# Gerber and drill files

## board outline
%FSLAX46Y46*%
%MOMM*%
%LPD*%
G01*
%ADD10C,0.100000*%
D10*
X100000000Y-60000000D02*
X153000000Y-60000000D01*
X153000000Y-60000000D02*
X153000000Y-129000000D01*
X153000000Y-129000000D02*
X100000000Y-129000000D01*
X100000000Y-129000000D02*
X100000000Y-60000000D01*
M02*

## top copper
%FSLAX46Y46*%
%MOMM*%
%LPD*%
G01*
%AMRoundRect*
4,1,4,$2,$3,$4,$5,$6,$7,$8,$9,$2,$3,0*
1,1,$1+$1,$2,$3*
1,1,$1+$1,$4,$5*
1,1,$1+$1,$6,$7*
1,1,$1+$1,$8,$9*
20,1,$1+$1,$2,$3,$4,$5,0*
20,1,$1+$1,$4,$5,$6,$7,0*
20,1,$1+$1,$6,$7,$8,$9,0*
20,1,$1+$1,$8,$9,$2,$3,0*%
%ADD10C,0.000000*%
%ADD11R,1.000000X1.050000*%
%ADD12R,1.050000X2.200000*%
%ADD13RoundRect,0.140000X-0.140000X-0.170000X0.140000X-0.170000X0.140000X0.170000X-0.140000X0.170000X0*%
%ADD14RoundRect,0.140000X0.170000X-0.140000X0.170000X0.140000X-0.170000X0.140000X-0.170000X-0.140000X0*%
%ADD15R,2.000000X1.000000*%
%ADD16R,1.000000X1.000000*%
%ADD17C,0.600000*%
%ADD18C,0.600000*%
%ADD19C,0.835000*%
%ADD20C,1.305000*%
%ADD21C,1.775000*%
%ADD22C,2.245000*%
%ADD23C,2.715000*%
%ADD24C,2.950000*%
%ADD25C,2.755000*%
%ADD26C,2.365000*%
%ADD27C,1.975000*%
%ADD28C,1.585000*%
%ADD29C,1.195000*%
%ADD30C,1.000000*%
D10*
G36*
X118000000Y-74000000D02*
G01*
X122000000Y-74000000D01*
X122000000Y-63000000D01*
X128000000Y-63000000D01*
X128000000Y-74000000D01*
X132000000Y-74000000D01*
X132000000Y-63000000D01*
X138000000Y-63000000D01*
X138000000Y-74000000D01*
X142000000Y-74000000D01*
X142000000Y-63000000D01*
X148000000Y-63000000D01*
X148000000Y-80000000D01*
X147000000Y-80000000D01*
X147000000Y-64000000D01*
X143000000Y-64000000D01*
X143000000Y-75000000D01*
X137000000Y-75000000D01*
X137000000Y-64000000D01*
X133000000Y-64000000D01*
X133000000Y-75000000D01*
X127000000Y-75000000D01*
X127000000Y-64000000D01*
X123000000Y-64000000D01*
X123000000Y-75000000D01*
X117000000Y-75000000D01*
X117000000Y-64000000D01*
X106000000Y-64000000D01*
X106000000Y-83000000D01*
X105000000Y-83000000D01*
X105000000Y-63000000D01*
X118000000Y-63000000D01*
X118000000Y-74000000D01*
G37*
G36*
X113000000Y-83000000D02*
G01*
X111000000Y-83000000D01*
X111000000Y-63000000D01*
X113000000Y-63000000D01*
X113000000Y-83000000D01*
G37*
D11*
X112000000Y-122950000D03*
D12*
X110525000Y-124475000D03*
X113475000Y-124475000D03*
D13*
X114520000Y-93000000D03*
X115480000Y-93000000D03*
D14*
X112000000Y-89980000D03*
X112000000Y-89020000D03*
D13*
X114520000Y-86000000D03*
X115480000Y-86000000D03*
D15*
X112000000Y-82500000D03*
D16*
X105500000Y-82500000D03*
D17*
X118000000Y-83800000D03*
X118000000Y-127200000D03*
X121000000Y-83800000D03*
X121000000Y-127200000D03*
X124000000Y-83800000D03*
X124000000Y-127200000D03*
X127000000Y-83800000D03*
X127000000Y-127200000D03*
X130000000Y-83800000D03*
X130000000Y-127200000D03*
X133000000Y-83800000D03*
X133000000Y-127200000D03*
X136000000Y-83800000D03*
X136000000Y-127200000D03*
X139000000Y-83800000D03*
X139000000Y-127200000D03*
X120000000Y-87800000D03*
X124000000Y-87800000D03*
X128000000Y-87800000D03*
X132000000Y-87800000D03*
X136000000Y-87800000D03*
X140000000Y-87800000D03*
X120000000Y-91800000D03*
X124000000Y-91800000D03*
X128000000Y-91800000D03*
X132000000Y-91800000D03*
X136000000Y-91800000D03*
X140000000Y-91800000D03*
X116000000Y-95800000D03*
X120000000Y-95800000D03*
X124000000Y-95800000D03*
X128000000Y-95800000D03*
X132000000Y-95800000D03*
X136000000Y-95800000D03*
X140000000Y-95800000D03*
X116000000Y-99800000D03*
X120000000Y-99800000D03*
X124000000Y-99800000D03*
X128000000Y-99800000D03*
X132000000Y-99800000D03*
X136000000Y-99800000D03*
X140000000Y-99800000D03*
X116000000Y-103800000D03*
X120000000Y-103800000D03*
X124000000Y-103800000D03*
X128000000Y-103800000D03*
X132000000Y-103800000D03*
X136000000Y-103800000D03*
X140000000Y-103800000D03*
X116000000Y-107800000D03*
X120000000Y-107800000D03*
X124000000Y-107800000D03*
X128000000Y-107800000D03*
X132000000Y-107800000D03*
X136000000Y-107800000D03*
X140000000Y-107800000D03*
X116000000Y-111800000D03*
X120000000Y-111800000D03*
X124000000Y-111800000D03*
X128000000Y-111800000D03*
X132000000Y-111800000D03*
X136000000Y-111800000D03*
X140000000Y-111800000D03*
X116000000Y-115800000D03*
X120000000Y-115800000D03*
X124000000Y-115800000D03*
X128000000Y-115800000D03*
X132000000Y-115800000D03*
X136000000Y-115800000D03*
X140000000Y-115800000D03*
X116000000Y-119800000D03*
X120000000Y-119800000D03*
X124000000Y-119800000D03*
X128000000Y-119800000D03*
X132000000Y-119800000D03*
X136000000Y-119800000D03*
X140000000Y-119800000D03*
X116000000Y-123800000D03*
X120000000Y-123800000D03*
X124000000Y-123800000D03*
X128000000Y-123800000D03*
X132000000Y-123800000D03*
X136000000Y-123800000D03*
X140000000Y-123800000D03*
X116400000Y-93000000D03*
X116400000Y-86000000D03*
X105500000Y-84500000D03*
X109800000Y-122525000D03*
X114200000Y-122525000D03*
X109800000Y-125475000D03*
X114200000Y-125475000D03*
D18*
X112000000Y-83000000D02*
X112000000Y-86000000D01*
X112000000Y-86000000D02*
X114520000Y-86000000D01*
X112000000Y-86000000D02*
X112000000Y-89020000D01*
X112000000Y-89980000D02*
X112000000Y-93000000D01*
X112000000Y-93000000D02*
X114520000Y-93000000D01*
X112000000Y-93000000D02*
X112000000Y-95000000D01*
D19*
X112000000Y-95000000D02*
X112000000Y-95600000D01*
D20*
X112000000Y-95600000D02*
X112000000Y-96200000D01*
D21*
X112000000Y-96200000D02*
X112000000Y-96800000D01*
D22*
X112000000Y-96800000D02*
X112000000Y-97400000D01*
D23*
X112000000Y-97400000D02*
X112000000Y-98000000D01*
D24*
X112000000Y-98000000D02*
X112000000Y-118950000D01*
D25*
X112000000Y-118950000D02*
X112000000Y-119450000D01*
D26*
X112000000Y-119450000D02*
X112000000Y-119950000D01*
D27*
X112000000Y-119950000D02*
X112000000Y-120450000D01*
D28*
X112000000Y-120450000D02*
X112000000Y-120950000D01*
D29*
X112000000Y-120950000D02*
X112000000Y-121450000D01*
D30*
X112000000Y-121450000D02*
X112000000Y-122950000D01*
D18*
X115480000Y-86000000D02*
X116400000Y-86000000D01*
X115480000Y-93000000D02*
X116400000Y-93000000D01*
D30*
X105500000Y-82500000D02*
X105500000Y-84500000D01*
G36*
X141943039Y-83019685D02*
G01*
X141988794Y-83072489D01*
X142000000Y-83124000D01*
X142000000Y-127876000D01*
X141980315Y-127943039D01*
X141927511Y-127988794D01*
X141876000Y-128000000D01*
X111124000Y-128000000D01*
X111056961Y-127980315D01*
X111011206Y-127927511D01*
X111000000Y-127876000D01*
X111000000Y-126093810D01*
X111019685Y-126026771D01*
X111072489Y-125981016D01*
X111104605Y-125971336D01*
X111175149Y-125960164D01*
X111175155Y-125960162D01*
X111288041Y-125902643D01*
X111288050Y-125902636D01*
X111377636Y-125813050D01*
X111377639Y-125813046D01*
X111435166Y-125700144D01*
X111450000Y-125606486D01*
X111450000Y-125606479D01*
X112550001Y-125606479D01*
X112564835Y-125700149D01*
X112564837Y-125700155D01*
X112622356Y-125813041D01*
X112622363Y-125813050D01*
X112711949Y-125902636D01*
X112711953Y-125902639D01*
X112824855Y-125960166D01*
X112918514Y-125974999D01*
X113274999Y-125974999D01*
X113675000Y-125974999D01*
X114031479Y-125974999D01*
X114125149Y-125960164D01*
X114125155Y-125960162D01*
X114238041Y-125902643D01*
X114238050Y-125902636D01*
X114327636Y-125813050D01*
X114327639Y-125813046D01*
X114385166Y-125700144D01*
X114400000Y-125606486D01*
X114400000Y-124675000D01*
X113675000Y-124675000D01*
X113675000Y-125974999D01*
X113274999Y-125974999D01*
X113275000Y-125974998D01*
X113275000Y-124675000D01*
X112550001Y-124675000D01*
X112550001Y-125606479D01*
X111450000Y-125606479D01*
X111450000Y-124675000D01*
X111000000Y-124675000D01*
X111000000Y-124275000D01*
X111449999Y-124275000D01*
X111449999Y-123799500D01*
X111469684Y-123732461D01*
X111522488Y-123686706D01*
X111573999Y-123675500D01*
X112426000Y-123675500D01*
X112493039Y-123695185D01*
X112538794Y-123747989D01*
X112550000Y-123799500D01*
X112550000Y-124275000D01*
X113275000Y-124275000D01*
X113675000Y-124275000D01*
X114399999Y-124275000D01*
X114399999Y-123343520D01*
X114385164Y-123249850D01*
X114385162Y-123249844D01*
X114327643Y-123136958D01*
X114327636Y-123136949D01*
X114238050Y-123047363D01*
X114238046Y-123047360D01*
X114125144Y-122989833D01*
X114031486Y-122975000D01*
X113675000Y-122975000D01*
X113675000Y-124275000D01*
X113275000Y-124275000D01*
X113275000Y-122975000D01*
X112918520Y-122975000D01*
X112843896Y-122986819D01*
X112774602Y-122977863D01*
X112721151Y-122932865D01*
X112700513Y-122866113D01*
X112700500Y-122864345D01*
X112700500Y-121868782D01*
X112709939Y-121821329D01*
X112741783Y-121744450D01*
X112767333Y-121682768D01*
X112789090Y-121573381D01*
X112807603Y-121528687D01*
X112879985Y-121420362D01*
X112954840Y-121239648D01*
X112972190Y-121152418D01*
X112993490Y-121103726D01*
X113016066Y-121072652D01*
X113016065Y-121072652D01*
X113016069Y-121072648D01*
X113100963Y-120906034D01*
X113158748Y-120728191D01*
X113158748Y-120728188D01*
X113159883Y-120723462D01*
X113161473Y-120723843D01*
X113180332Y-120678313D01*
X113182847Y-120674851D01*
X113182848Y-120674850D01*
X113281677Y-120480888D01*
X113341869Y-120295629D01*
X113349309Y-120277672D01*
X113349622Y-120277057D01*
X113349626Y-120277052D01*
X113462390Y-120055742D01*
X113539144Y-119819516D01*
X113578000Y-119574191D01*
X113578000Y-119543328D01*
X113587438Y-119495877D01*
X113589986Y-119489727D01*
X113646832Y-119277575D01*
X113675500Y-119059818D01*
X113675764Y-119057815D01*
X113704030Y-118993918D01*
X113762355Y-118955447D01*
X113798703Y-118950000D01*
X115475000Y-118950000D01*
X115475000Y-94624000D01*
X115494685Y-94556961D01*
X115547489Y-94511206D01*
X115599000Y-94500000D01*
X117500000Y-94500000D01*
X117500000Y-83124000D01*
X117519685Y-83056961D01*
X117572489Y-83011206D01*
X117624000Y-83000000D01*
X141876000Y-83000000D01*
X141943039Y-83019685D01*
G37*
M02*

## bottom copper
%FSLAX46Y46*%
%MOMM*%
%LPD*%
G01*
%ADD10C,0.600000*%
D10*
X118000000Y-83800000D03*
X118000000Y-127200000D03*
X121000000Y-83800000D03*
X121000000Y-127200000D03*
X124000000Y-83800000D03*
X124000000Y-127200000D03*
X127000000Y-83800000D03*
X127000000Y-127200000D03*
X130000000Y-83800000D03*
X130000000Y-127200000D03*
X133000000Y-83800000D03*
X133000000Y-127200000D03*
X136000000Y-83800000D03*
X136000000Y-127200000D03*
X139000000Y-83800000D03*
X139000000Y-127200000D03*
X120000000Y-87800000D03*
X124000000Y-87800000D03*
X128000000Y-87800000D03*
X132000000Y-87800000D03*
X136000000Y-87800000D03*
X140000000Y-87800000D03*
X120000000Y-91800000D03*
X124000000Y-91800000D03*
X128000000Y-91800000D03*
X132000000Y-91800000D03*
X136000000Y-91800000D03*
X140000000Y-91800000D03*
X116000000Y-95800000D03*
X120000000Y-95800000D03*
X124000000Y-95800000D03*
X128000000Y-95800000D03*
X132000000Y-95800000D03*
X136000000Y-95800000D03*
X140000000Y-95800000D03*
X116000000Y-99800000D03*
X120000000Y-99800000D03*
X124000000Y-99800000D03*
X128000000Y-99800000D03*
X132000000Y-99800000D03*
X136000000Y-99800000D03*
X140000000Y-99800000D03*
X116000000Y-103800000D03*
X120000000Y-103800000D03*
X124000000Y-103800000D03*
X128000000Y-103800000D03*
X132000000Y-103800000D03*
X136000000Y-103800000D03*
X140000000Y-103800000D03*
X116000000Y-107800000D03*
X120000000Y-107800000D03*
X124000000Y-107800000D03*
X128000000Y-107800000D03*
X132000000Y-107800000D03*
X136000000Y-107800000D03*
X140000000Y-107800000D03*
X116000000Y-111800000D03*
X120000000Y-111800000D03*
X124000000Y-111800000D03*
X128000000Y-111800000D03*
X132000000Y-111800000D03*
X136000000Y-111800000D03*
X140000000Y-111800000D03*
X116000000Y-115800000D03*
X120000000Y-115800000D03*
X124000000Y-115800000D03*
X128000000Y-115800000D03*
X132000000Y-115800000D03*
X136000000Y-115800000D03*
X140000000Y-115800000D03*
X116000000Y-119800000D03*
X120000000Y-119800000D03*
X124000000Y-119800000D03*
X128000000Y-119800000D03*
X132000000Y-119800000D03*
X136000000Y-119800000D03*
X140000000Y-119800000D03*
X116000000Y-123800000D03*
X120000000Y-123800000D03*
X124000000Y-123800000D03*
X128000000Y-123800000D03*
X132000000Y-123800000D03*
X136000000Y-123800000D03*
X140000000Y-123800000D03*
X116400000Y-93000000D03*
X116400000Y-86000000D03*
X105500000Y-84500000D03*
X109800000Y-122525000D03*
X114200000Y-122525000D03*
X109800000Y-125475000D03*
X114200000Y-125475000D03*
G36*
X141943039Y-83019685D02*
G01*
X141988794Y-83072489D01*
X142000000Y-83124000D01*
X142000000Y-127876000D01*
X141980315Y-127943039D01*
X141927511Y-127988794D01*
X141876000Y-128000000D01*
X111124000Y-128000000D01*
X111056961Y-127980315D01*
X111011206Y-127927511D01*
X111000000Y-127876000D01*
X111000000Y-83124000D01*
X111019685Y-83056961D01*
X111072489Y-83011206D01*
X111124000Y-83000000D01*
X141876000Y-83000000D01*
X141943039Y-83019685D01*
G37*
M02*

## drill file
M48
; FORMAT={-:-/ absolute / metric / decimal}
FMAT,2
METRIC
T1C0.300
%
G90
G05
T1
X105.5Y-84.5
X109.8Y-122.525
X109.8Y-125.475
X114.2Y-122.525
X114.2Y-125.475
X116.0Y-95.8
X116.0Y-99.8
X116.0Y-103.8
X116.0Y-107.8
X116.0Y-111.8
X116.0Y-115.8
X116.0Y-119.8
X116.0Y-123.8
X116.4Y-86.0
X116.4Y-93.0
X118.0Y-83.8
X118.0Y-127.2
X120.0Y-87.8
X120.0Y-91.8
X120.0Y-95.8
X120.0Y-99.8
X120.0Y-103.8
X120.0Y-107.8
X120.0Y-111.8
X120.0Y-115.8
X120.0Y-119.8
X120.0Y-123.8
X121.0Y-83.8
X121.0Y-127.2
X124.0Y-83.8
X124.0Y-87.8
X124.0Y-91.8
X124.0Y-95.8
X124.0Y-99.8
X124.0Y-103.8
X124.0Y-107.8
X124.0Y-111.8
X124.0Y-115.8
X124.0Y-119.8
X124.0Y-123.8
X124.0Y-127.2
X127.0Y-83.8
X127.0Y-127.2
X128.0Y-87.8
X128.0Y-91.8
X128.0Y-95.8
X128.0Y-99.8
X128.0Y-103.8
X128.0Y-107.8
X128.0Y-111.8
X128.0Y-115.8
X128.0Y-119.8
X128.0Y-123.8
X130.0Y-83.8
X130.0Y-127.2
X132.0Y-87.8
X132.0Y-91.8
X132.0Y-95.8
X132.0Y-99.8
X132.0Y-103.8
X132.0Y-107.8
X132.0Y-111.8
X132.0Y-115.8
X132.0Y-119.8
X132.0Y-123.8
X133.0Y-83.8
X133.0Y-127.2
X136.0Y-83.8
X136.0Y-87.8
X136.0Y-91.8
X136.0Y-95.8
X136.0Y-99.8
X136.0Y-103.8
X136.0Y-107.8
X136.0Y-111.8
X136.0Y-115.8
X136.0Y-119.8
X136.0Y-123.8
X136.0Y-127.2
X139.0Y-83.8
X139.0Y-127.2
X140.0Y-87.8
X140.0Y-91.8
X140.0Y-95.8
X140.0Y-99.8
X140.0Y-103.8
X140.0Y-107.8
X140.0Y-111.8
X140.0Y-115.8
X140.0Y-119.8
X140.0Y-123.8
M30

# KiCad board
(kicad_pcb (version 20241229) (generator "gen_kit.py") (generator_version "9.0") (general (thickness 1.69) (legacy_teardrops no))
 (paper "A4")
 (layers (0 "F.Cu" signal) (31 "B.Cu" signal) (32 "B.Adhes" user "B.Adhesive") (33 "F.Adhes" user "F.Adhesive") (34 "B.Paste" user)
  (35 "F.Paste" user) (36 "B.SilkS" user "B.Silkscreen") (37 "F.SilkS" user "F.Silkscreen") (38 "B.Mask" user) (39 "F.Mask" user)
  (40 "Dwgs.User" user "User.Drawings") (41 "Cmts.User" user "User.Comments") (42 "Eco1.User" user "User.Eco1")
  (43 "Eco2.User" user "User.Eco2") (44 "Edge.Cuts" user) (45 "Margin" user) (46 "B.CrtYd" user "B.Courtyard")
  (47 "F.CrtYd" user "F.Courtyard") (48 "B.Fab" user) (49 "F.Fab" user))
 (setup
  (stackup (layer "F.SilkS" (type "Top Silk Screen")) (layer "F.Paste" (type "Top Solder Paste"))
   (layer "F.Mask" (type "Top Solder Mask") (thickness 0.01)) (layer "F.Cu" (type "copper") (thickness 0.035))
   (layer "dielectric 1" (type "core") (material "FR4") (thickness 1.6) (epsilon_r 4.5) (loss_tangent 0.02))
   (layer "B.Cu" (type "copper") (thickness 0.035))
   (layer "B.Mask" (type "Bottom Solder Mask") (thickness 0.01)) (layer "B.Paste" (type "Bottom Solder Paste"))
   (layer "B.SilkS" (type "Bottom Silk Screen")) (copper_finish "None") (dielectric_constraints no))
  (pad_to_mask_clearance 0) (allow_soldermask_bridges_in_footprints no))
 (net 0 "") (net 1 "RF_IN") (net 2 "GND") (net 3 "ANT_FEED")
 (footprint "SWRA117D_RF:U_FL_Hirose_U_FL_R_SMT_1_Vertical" (layer "F.Cu") (at 112 124 270)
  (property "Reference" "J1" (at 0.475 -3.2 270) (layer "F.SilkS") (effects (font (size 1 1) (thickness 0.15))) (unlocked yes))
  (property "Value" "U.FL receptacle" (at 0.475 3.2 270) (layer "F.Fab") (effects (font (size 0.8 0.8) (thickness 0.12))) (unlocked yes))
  (pad "1" smd rect (at -1.05 0 270) (size 1.05 1) (layers "F.Cu" "F.Paste" "F.Mask") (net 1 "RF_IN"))
  (pad "2" smd rect (at 0.475 1.475 270) (size 2.2 1.05) (layers "F.Cu" "F.Paste" "F.Mask") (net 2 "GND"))
  (pad "2" smd rect (at 0.475 -1.475 270) (size 2.2 1.05) (layers "F.Cu" "F.Paste" "F.Mask") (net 2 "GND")))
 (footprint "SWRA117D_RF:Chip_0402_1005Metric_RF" (layer "F.Cu") (at 115 93)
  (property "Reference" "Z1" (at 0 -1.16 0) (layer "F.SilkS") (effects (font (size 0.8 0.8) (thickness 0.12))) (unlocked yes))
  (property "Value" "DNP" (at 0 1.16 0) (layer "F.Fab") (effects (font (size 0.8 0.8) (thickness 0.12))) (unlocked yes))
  (pad "1" smd roundrect (at -0.48 0) (size 0.56 0.62) (layers "F.Cu" "F.Paste" "F.Mask") (roundrect_rratio 0.25) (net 1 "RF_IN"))
  (pad "2" smd roundrect (at 0.48 0) (size 0.56 0.62) (layers "F.Cu" "F.Paste" "F.Mask") (roundrect_rratio 0.25) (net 2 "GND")))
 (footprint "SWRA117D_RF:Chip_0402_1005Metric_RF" (layer "F.Cu") (at 112 89.5 90)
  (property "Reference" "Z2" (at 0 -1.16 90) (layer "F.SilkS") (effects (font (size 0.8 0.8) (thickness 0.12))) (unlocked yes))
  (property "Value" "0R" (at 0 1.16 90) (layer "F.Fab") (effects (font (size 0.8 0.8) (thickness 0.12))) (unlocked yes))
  (pad "1" smd roundrect (at -0.48 0 90) (size 0.56 0.62) (layers "F.Cu" "F.Paste" "F.Mask") (roundrect_rratio 0.25) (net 1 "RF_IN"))
  (pad "2" smd roundrect (at 0.48 0 90) (size 0.56 0.62) (layers "F.Cu" "F.Paste" "F.Mask") (roundrect_rratio 0.25) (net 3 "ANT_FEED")))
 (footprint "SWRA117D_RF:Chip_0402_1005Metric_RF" (layer "F.Cu") (at 115 86)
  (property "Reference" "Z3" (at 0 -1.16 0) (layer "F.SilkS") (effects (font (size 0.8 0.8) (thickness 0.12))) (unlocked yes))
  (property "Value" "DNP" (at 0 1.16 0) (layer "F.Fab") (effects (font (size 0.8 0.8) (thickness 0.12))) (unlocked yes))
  (pad "1" smd roundrect (at -0.48 0) (size 0.56 0.62) (layers "F.Cu" "F.Paste" "F.Mask") (roundrect_rratio 0.25) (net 3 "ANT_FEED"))
  (pad "2" smd roundrect (at 0.48 0) (size 0.56 0.62) (layers "F.Cu" "F.Paste" "F.Mask") (roundrect_rratio 0.25) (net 2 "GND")))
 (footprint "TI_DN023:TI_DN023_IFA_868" (layer "F.Cu") (at 112 83)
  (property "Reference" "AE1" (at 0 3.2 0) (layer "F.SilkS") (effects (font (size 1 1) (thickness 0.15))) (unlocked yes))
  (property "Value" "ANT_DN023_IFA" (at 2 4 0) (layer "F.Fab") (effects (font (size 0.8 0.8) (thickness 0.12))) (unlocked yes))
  (fp_poly
   (pts (xy -6 0) (xy -6 -19) (xy 5 -19) (xy 5 -8) (xy 11 -8) (xy 11 -19) (xy 15 -19) (xy 15 -8) (xy 21 -8) (xy 21 -19) (xy 25 -19)
    (xy 25 -8) (xy 31 -8) (xy 31 -19) (xy 35 -19) (xy 35 -3) (xy 36 -3) (xy 36 -20) (xy 30 -20) (xy 30 -9) (xy 26 -9) (xy 26 -20)
    (xy 20 -20) (xy 20 -9) (xy 16 -9) (xy 16 -20) (xy 10 -20) (xy 10 -9) (xy 6 -9) (xy 6 -20) (xy -7 -20) (xy -7 0))
   (stroke (width 0) (type solid)) (fill yes) (layer "F.Cu"))
  (fp_poly (pts (xy 1 0) (xy 1 -20) (xy -1 -20) (xy -1 0)) (stroke (width 0) (type solid)) (fill yes) (layer "F.Cu"))
  (pad "1" smd rect (at 0 -0.5) (size 2 1) (layers "F.Cu" "F.Mask") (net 3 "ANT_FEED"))
  (pad "2" smd rect (at -6.5 -0.5) (size 1 1) (layers "F.Cu" "F.Mask") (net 2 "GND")))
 (gr_line (start 100 60) (end 153 60) (stroke (width 0.1) (type solid)) (layer "Edge.Cuts"))
 (gr_line (start 153 60) (end 153 129) (stroke (width 0.1) (type solid)) (layer "Edge.Cuts"))
 (gr_line (start 153 129) (end 100 129) (stroke (width 0.1) (type solid)) (layer "Edge.Cuts"))
 (gr_line (start 100 129) (end 100 60) (stroke (width 0.1) (type solid)) (layer "Edge.Cuts"))
 (segment (start 112 83) (end 112 86) (width 0.6) (layer "F.Cu") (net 3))
 (segment (start 112 86) (end 114.52 86) (width 0.6) (layer "F.Cu") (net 3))
 (segment (start 112 86) (end 112 89.02) (width 0.6) (layer "F.Cu") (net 3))
 (segment (start 112 89.98) (end 112 93) (width 0.6) (layer "F.Cu") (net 1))
 (segment (start 112 93) (end 114.52 93) (width 0.6) (layer "F.Cu") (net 1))
 (segment (start 112 93) (end 112 95) (width 0.6) (layer "F.Cu") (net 1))
 (segment (start 112 95) (end 112 95.6) (width 0.835) (layer "F.Cu") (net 1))
 (segment (start 112 95.6) (end 112 96.2) (width 1.305) (layer "F.Cu") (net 1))
 (segment (start 112 96.2) (end 112 96.8) (width 1.775) (layer "F.Cu") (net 1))
 (segment (start 112 96.8) (end 112 97.4) (width 2.245) (layer "F.Cu") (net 1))
 (segment (start 112 97.4) (end 112 98) (width 2.715) (layer "F.Cu") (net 1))
 (segment (start 112 98) (end 112 118.95) (width 2.95) (layer "F.Cu") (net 1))
 (segment (start 112 118.95) (end 112 119.45) (width 2.755) (layer "F.Cu") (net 1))
 (segment (start 112 119.45) (end 112 119.95) (width 2.365) (layer "F.Cu") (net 1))
 (segment (start 112 119.95) (end 112 120.45) (width 1.975) (layer "F.Cu") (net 1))
 (segment (start 112 120.45) (end 112 120.95) (width 1.585) (layer "F.Cu") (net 1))
 (segment (start 112 120.95) (end 112 121.45) (width 1.195) (layer "F.Cu") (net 1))
 (segment (start 112 121.45) (end 112 122.95) (width 1) (layer "F.Cu") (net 1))
 (segment (start 115.48 86) (end 116.4 86) (width 0.6) (layer "F.Cu") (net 2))
 (segment (start 115.48 93) (end 116.4 93) (width 0.6) (layer "F.Cu") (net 2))
 (segment (start 105.5 82.5) (end 105.5 84.5) (width 1) (layer "F.Cu") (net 2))
 (via (at 118 83.8) (size 0.6) (drill 0.3) (layers "F.Cu" "B.Cu") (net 2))
 (via (at 118 127.2) (size 0.6) (drill 0.3) (layers "F.Cu" "B.Cu") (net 2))
 (via (at 121 83.8) (size 0.6) (drill 0.3) (layers "F.Cu" "B.Cu") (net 2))
 (via (at 121 127.2) (size 0.6) (drill 0.3) (layers "F.Cu" "B.Cu") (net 2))
 (via (at 124 83.8) (size 0.6) (drill 0.3) (layers "F.Cu" "B.Cu") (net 2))
 (via (at 124 127.2) (size 0.6) (drill 0.3) (layers "F.Cu" "B.Cu") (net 2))
 (via (at 127 83.8) (size 0.6) (drill 0.3) (layers "F.Cu" "B.Cu") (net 2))
 (via (at 127 127.2) (size 0.6) (drill 0.3) (layers "F.Cu" "B.Cu") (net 2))
 (via (at 130 83.8) (size 0.6) (drill 0.3) (layers "F.Cu" "B.Cu") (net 2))
 (via (at 130 127.2) (size 0.6) (drill 0.3) (layers "F.Cu" "B.Cu") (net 2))
 (via (at 133 83.8) (size 0.6) (drill 0.3) (layers "F.Cu" "B.Cu") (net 2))
 (via (at 133 127.2) (size 0.6) (drill 0.3) (layers "F.Cu" "B.Cu") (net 2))
 (via (at 136 83.8) (size 0.6) (drill 0.3) (layers "F.Cu" "B.Cu") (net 2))
 (via (at 136 127.2) (size 0.6) (drill 0.3) (layers "F.Cu" "B.Cu") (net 2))
 (via (at 139 83.8) (size 0.6) (drill 0.3) (layers "F.Cu" "B.Cu") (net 2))
 (via (at 139 127.2) (size 0.6) (drill 0.3) (layers "F.Cu" "B.Cu") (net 2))
 (via (at 120 87.8) (size 0.6) (drill 0.3) (layers "F.Cu" "B.Cu") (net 2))
 (via (at 124 87.8) (size 0.6) (drill 0.3) (layers "F.Cu" "B.Cu") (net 2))
 (via (at 128 87.8) (size 0.6) (drill 0.3) (layers "F.Cu" "B.Cu") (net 2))
 (via (at 132 87.8) (size 0.6) (drill 0.3) (layers "F.Cu" "B.Cu") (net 2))
 (via (at 136 87.8) (size 0.6) (drill 0.3) (layers "F.Cu" "B.Cu") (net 2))
 (via (at 140 87.8) (size 0.6) (drill 0.3) (layers "F.Cu" "B.Cu") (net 2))
 (via (at 120 91.8) (size 0.6) (drill 0.3) (layers "F.Cu" "B.Cu") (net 2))
 (via (at 124 91.8) (size 0.6) (drill 0.3) (layers "F.Cu" "B.Cu") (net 2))
 (via (at 128 91.8) (size 0.6) (drill 0.3) (layers "F.Cu" "B.Cu") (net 2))
 (via (at 132 91.8) (size 0.6) (drill 0.3) (layers "F.Cu" "B.Cu") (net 2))
 (via (at 136 91.8) (size 0.6) (drill 0.3) (layers "F.Cu" "B.Cu") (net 2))
 (via (at 140 91.8) (size 0.6) (drill 0.3) (layers "F.Cu" "B.Cu") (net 2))
 (via (at 116 95.8) (size 0.6) (drill 0.3) (layers "F.Cu" "B.Cu") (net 2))
 (via (at 120 95.8) (size 0.6) (drill 0.3) (layers "F.Cu" "B.Cu") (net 2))
 (via (at 124 95.8) (size 0.6) (drill 0.3) (layers "F.Cu" "B.Cu") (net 2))
 (via (at 128 95.8) (size 0.6) (drill 0.3) (layers "F.Cu" "B.Cu") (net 2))
 (via (at 132 95.8) (size 0.6) (drill 0.3) (layers "F.Cu" "B.Cu") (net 2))
 (via (at 136 95.8) (size 0.6) (drill 0.3) (layers "F.Cu" "B.Cu") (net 2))
 (via (at 140 95.8) (size 0.6) (drill 0.3) (layers "F.Cu" "B.Cu") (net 2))
 (via (at 116 99.8) (size 0.6) (drill 0.3) (layers "F.Cu" "B.Cu") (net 2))
 (via (at 120 99.8) (size 0.6) (drill 0.3) (layers "F.Cu" "B.Cu") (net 2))
 (via (at 124 99.8) (size 0.6) (drill 0.3) (layers "F.Cu" "B.Cu") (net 2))
 (via (at 128 99.8) (size 0.6) (drill 0.3) (layers "F.Cu" "B.Cu") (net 2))
 (via (at 132 99.8) (size 0.6) (drill 0.3) (layers "F.Cu" "B.Cu") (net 2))
 (via (at 136 99.8) (size 0.6) (drill 0.3) (layers "F.Cu" "B.Cu") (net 2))
 (via (at 140 99.8) (size 0.6) (drill 0.3) (layers "F.Cu" "B.Cu") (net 2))
 (via (at 116 103.8) (size 0.6) (drill 0.3) (layers "F.Cu" "B.Cu") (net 2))
 (via (at 120 103.8) (size 0.6) (drill 0.3) (layers "F.Cu" "B.Cu") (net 2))
 (via (at 124 103.8) (size 0.6) (drill 0.3) (layers "F.Cu" "B.Cu") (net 2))
 (via (at 128 103.8) (size 0.6) (drill 0.3) (layers "F.Cu" "B.Cu") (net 2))
 (via (at 132 103.8) (size 0.6) (drill 0.3) (layers "F.Cu" "B.Cu") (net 2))
 (via (at 136 103.8) (size 0.6) (drill 0.3) (layers "F.Cu" "B.Cu") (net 2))
 (via (at 140 103.8) (size 0.6) (drill 0.3) (layers "F.Cu" "B.Cu") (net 2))
 (via (at 116 107.8) (size 0.6) (drill 0.3) (layers "F.Cu" "B.Cu") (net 2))
 (via (at 120 107.8) (size 0.6) (drill 0.3) (layers "F.Cu" "B.Cu") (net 2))
 (via (at 124 107.8) (size 0.6) (drill 0.3) (layers "F.Cu" "B.Cu") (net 2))
 (via (at 128 107.8) (size 0.6) (drill 0.3) (layers "F.Cu" "B.Cu") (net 2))
 (via (at 132 107.8) (size 0.6) (drill 0.3) (layers "F.Cu" "B.Cu") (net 2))
 (via (at 136 107.8) (size 0.6) (drill 0.3) (layers "F.Cu" "B.Cu") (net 2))
 (via (at 140 107.8) (size 0.6) (drill 0.3) (layers "F.Cu" "B.Cu") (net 2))
 (via (at 116 111.8) (size 0.6) (drill 0.3) (layers "F.Cu" "B.Cu") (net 2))
 (via (at 120 111.8) (size 0.6) (drill 0.3) (layers "F.Cu" "B.Cu") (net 2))
 (via (at 124 111.8) (size 0.6) (drill 0.3) (layers "F.Cu" "B.Cu") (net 2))
 (via (at 128 111.8) (size 0.6) (drill 0.3) (layers "F.Cu" "B.Cu") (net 2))
 (via (at 132 111.8) (size 0.6) (drill 0.3) (layers "F.Cu" "B.Cu") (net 2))
 (via (at 136 111.8) (size 0.6) (drill 0.3) (layers "F.Cu" "B.Cu") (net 2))
 (via (at 140 111.8) (size 0.6) (drill 0.3) (layers "F.Cu" "B.Cu") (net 2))
 (via (at 116 115.8) (size 0.6) (drill 0.3) (layers "F.Cu" "B.Cu") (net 2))
 (via (at 120 115.8) (size 0.6) (drill 0.3) (layers "F.Cu" "B.Cu") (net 2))
 (via (at 124 115.8) (size 0.6) (drill 0.3) (layers "F.Cu" "B.Cu") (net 2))
 (via (at 128 115.8) (size 0.6) (drill 0.3) (layers "F.Cu" "B.Cu") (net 2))
 (via (at 132 115.8) (size 0.6) (drill 0.3) (layers "F.Cu" "B.Cu") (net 2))
 (via (at 136 115.8) (size 0.6) (drill 0.3) (layers "F.Cu" "B.Cu") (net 2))
 (via (at 140 115.8) (size 0.6) (drill 0.3) (layers "F.Cu" "B.Cu") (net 2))
 (via (at 116 119.8) (size 0.6) (drill 0.3) (layers "F.Cu" "B.Cu") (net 2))
 (via (at 120 119.8) (size 0.6) (drill 0.3) (layers "F.Cu" "B.Cu") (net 2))
 (via (at 124 119.8) (size 0.6) (drill 0.3) (layers "F.Cu" "B.Cu") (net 2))
 (via (at 128 119.8) (size 0.6) (drill 0.3) (layers "F.Cu" "B.Cu") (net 2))
 (via (at 132 119.8) (size 0.6) (drill 0.3) (layers "F.Cu" "B.Cu") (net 2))
 (via (at 136 119.8) (size 0.6) (drill 0.3) (layers "F.Cu" "B.Cu") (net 2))
 (via (at 140 119.8) (size 0.6) (drill 0.3) (layers "F.Cu" "B.Cu") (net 2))
 (via (at 116 123.8) (size 0.6) (drill 0.3) (layers "F.Cu" "B.Cu") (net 2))
 (via (at 120 123.8) (size 0.6) (drill 0.3) (layers "F.Cu" "B.Cu") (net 2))
 (via (at 124 123.8) (size 0.6) (drill 0.3) (layers "F.Cu" "B.Cu") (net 2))
 (via (at 128 123.8) (size 0.6) (drill 0.3) (layers "F.Cu" "B.Cu") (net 2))
 (via (at 132 123.8) (size 0.6) (drill 0.3) (layers "F.Cu" "B.Cu") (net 2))
 (via (at 136 123.8) (size 0.6) (drill 0.3) (layers "F.Cu" "B.Cu") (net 2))
 (via (at 140 123.8) (size 0.6) (drill 0.3) (layers "F.Cu" "B.Cu") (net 2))
 (via (at 116.4 93) (size 0.6) (drill 0.3) (layers "F.Cu" "B.Cu") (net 2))
 (via (at 116.4 86) (size 0.6) (drill 0.3) (layers "F.Cu" "B.Cu") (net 2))
 (via (at 105.5 84.5) (size 0.6) (drill 0.3) (layers "F.Cu" "B.Cu") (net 2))
 (via (at 109.8 122.525) (size 0.6) (drill 0.3) (layers "F.Cu" "B.Cu") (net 2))
 (via (at 114.2 122.525) (size 0.6) (drill 0.3) (layers "F.Cu" "B.Cu") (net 2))
 (via (at 109.8 125.475) (size 0.6) (drill 0.3) (layers "F.Cu" "B.Cu") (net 2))
 (via (at 114.2 125.475) (size 0.6) (drill 0.3) (layers "F.Cu" "B.Cu") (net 2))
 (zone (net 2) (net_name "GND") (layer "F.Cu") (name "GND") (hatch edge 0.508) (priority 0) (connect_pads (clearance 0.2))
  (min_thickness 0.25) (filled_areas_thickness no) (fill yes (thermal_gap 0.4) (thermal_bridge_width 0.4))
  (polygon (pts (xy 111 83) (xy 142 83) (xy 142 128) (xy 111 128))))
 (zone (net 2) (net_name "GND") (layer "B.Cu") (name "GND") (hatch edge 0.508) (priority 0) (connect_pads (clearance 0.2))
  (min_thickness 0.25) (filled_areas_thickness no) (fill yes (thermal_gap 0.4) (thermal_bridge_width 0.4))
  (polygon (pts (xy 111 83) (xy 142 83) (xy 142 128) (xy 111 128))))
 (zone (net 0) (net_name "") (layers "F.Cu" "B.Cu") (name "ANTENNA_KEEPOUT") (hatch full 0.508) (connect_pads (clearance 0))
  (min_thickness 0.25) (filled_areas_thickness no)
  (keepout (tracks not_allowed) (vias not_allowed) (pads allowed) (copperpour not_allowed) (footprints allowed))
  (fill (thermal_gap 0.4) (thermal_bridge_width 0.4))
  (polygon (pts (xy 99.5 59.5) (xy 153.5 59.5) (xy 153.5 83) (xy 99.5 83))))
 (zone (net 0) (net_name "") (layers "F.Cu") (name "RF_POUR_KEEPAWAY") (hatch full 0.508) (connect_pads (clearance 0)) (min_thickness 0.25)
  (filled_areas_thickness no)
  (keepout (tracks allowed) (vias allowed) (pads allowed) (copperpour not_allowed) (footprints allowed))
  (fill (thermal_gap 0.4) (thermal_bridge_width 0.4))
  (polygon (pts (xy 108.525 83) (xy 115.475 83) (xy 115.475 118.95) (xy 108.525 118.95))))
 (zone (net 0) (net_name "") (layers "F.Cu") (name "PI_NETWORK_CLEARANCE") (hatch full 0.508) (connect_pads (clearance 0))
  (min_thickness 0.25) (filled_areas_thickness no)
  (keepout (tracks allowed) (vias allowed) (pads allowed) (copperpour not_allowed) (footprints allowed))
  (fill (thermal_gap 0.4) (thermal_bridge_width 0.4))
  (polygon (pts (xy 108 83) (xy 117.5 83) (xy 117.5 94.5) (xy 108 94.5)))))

